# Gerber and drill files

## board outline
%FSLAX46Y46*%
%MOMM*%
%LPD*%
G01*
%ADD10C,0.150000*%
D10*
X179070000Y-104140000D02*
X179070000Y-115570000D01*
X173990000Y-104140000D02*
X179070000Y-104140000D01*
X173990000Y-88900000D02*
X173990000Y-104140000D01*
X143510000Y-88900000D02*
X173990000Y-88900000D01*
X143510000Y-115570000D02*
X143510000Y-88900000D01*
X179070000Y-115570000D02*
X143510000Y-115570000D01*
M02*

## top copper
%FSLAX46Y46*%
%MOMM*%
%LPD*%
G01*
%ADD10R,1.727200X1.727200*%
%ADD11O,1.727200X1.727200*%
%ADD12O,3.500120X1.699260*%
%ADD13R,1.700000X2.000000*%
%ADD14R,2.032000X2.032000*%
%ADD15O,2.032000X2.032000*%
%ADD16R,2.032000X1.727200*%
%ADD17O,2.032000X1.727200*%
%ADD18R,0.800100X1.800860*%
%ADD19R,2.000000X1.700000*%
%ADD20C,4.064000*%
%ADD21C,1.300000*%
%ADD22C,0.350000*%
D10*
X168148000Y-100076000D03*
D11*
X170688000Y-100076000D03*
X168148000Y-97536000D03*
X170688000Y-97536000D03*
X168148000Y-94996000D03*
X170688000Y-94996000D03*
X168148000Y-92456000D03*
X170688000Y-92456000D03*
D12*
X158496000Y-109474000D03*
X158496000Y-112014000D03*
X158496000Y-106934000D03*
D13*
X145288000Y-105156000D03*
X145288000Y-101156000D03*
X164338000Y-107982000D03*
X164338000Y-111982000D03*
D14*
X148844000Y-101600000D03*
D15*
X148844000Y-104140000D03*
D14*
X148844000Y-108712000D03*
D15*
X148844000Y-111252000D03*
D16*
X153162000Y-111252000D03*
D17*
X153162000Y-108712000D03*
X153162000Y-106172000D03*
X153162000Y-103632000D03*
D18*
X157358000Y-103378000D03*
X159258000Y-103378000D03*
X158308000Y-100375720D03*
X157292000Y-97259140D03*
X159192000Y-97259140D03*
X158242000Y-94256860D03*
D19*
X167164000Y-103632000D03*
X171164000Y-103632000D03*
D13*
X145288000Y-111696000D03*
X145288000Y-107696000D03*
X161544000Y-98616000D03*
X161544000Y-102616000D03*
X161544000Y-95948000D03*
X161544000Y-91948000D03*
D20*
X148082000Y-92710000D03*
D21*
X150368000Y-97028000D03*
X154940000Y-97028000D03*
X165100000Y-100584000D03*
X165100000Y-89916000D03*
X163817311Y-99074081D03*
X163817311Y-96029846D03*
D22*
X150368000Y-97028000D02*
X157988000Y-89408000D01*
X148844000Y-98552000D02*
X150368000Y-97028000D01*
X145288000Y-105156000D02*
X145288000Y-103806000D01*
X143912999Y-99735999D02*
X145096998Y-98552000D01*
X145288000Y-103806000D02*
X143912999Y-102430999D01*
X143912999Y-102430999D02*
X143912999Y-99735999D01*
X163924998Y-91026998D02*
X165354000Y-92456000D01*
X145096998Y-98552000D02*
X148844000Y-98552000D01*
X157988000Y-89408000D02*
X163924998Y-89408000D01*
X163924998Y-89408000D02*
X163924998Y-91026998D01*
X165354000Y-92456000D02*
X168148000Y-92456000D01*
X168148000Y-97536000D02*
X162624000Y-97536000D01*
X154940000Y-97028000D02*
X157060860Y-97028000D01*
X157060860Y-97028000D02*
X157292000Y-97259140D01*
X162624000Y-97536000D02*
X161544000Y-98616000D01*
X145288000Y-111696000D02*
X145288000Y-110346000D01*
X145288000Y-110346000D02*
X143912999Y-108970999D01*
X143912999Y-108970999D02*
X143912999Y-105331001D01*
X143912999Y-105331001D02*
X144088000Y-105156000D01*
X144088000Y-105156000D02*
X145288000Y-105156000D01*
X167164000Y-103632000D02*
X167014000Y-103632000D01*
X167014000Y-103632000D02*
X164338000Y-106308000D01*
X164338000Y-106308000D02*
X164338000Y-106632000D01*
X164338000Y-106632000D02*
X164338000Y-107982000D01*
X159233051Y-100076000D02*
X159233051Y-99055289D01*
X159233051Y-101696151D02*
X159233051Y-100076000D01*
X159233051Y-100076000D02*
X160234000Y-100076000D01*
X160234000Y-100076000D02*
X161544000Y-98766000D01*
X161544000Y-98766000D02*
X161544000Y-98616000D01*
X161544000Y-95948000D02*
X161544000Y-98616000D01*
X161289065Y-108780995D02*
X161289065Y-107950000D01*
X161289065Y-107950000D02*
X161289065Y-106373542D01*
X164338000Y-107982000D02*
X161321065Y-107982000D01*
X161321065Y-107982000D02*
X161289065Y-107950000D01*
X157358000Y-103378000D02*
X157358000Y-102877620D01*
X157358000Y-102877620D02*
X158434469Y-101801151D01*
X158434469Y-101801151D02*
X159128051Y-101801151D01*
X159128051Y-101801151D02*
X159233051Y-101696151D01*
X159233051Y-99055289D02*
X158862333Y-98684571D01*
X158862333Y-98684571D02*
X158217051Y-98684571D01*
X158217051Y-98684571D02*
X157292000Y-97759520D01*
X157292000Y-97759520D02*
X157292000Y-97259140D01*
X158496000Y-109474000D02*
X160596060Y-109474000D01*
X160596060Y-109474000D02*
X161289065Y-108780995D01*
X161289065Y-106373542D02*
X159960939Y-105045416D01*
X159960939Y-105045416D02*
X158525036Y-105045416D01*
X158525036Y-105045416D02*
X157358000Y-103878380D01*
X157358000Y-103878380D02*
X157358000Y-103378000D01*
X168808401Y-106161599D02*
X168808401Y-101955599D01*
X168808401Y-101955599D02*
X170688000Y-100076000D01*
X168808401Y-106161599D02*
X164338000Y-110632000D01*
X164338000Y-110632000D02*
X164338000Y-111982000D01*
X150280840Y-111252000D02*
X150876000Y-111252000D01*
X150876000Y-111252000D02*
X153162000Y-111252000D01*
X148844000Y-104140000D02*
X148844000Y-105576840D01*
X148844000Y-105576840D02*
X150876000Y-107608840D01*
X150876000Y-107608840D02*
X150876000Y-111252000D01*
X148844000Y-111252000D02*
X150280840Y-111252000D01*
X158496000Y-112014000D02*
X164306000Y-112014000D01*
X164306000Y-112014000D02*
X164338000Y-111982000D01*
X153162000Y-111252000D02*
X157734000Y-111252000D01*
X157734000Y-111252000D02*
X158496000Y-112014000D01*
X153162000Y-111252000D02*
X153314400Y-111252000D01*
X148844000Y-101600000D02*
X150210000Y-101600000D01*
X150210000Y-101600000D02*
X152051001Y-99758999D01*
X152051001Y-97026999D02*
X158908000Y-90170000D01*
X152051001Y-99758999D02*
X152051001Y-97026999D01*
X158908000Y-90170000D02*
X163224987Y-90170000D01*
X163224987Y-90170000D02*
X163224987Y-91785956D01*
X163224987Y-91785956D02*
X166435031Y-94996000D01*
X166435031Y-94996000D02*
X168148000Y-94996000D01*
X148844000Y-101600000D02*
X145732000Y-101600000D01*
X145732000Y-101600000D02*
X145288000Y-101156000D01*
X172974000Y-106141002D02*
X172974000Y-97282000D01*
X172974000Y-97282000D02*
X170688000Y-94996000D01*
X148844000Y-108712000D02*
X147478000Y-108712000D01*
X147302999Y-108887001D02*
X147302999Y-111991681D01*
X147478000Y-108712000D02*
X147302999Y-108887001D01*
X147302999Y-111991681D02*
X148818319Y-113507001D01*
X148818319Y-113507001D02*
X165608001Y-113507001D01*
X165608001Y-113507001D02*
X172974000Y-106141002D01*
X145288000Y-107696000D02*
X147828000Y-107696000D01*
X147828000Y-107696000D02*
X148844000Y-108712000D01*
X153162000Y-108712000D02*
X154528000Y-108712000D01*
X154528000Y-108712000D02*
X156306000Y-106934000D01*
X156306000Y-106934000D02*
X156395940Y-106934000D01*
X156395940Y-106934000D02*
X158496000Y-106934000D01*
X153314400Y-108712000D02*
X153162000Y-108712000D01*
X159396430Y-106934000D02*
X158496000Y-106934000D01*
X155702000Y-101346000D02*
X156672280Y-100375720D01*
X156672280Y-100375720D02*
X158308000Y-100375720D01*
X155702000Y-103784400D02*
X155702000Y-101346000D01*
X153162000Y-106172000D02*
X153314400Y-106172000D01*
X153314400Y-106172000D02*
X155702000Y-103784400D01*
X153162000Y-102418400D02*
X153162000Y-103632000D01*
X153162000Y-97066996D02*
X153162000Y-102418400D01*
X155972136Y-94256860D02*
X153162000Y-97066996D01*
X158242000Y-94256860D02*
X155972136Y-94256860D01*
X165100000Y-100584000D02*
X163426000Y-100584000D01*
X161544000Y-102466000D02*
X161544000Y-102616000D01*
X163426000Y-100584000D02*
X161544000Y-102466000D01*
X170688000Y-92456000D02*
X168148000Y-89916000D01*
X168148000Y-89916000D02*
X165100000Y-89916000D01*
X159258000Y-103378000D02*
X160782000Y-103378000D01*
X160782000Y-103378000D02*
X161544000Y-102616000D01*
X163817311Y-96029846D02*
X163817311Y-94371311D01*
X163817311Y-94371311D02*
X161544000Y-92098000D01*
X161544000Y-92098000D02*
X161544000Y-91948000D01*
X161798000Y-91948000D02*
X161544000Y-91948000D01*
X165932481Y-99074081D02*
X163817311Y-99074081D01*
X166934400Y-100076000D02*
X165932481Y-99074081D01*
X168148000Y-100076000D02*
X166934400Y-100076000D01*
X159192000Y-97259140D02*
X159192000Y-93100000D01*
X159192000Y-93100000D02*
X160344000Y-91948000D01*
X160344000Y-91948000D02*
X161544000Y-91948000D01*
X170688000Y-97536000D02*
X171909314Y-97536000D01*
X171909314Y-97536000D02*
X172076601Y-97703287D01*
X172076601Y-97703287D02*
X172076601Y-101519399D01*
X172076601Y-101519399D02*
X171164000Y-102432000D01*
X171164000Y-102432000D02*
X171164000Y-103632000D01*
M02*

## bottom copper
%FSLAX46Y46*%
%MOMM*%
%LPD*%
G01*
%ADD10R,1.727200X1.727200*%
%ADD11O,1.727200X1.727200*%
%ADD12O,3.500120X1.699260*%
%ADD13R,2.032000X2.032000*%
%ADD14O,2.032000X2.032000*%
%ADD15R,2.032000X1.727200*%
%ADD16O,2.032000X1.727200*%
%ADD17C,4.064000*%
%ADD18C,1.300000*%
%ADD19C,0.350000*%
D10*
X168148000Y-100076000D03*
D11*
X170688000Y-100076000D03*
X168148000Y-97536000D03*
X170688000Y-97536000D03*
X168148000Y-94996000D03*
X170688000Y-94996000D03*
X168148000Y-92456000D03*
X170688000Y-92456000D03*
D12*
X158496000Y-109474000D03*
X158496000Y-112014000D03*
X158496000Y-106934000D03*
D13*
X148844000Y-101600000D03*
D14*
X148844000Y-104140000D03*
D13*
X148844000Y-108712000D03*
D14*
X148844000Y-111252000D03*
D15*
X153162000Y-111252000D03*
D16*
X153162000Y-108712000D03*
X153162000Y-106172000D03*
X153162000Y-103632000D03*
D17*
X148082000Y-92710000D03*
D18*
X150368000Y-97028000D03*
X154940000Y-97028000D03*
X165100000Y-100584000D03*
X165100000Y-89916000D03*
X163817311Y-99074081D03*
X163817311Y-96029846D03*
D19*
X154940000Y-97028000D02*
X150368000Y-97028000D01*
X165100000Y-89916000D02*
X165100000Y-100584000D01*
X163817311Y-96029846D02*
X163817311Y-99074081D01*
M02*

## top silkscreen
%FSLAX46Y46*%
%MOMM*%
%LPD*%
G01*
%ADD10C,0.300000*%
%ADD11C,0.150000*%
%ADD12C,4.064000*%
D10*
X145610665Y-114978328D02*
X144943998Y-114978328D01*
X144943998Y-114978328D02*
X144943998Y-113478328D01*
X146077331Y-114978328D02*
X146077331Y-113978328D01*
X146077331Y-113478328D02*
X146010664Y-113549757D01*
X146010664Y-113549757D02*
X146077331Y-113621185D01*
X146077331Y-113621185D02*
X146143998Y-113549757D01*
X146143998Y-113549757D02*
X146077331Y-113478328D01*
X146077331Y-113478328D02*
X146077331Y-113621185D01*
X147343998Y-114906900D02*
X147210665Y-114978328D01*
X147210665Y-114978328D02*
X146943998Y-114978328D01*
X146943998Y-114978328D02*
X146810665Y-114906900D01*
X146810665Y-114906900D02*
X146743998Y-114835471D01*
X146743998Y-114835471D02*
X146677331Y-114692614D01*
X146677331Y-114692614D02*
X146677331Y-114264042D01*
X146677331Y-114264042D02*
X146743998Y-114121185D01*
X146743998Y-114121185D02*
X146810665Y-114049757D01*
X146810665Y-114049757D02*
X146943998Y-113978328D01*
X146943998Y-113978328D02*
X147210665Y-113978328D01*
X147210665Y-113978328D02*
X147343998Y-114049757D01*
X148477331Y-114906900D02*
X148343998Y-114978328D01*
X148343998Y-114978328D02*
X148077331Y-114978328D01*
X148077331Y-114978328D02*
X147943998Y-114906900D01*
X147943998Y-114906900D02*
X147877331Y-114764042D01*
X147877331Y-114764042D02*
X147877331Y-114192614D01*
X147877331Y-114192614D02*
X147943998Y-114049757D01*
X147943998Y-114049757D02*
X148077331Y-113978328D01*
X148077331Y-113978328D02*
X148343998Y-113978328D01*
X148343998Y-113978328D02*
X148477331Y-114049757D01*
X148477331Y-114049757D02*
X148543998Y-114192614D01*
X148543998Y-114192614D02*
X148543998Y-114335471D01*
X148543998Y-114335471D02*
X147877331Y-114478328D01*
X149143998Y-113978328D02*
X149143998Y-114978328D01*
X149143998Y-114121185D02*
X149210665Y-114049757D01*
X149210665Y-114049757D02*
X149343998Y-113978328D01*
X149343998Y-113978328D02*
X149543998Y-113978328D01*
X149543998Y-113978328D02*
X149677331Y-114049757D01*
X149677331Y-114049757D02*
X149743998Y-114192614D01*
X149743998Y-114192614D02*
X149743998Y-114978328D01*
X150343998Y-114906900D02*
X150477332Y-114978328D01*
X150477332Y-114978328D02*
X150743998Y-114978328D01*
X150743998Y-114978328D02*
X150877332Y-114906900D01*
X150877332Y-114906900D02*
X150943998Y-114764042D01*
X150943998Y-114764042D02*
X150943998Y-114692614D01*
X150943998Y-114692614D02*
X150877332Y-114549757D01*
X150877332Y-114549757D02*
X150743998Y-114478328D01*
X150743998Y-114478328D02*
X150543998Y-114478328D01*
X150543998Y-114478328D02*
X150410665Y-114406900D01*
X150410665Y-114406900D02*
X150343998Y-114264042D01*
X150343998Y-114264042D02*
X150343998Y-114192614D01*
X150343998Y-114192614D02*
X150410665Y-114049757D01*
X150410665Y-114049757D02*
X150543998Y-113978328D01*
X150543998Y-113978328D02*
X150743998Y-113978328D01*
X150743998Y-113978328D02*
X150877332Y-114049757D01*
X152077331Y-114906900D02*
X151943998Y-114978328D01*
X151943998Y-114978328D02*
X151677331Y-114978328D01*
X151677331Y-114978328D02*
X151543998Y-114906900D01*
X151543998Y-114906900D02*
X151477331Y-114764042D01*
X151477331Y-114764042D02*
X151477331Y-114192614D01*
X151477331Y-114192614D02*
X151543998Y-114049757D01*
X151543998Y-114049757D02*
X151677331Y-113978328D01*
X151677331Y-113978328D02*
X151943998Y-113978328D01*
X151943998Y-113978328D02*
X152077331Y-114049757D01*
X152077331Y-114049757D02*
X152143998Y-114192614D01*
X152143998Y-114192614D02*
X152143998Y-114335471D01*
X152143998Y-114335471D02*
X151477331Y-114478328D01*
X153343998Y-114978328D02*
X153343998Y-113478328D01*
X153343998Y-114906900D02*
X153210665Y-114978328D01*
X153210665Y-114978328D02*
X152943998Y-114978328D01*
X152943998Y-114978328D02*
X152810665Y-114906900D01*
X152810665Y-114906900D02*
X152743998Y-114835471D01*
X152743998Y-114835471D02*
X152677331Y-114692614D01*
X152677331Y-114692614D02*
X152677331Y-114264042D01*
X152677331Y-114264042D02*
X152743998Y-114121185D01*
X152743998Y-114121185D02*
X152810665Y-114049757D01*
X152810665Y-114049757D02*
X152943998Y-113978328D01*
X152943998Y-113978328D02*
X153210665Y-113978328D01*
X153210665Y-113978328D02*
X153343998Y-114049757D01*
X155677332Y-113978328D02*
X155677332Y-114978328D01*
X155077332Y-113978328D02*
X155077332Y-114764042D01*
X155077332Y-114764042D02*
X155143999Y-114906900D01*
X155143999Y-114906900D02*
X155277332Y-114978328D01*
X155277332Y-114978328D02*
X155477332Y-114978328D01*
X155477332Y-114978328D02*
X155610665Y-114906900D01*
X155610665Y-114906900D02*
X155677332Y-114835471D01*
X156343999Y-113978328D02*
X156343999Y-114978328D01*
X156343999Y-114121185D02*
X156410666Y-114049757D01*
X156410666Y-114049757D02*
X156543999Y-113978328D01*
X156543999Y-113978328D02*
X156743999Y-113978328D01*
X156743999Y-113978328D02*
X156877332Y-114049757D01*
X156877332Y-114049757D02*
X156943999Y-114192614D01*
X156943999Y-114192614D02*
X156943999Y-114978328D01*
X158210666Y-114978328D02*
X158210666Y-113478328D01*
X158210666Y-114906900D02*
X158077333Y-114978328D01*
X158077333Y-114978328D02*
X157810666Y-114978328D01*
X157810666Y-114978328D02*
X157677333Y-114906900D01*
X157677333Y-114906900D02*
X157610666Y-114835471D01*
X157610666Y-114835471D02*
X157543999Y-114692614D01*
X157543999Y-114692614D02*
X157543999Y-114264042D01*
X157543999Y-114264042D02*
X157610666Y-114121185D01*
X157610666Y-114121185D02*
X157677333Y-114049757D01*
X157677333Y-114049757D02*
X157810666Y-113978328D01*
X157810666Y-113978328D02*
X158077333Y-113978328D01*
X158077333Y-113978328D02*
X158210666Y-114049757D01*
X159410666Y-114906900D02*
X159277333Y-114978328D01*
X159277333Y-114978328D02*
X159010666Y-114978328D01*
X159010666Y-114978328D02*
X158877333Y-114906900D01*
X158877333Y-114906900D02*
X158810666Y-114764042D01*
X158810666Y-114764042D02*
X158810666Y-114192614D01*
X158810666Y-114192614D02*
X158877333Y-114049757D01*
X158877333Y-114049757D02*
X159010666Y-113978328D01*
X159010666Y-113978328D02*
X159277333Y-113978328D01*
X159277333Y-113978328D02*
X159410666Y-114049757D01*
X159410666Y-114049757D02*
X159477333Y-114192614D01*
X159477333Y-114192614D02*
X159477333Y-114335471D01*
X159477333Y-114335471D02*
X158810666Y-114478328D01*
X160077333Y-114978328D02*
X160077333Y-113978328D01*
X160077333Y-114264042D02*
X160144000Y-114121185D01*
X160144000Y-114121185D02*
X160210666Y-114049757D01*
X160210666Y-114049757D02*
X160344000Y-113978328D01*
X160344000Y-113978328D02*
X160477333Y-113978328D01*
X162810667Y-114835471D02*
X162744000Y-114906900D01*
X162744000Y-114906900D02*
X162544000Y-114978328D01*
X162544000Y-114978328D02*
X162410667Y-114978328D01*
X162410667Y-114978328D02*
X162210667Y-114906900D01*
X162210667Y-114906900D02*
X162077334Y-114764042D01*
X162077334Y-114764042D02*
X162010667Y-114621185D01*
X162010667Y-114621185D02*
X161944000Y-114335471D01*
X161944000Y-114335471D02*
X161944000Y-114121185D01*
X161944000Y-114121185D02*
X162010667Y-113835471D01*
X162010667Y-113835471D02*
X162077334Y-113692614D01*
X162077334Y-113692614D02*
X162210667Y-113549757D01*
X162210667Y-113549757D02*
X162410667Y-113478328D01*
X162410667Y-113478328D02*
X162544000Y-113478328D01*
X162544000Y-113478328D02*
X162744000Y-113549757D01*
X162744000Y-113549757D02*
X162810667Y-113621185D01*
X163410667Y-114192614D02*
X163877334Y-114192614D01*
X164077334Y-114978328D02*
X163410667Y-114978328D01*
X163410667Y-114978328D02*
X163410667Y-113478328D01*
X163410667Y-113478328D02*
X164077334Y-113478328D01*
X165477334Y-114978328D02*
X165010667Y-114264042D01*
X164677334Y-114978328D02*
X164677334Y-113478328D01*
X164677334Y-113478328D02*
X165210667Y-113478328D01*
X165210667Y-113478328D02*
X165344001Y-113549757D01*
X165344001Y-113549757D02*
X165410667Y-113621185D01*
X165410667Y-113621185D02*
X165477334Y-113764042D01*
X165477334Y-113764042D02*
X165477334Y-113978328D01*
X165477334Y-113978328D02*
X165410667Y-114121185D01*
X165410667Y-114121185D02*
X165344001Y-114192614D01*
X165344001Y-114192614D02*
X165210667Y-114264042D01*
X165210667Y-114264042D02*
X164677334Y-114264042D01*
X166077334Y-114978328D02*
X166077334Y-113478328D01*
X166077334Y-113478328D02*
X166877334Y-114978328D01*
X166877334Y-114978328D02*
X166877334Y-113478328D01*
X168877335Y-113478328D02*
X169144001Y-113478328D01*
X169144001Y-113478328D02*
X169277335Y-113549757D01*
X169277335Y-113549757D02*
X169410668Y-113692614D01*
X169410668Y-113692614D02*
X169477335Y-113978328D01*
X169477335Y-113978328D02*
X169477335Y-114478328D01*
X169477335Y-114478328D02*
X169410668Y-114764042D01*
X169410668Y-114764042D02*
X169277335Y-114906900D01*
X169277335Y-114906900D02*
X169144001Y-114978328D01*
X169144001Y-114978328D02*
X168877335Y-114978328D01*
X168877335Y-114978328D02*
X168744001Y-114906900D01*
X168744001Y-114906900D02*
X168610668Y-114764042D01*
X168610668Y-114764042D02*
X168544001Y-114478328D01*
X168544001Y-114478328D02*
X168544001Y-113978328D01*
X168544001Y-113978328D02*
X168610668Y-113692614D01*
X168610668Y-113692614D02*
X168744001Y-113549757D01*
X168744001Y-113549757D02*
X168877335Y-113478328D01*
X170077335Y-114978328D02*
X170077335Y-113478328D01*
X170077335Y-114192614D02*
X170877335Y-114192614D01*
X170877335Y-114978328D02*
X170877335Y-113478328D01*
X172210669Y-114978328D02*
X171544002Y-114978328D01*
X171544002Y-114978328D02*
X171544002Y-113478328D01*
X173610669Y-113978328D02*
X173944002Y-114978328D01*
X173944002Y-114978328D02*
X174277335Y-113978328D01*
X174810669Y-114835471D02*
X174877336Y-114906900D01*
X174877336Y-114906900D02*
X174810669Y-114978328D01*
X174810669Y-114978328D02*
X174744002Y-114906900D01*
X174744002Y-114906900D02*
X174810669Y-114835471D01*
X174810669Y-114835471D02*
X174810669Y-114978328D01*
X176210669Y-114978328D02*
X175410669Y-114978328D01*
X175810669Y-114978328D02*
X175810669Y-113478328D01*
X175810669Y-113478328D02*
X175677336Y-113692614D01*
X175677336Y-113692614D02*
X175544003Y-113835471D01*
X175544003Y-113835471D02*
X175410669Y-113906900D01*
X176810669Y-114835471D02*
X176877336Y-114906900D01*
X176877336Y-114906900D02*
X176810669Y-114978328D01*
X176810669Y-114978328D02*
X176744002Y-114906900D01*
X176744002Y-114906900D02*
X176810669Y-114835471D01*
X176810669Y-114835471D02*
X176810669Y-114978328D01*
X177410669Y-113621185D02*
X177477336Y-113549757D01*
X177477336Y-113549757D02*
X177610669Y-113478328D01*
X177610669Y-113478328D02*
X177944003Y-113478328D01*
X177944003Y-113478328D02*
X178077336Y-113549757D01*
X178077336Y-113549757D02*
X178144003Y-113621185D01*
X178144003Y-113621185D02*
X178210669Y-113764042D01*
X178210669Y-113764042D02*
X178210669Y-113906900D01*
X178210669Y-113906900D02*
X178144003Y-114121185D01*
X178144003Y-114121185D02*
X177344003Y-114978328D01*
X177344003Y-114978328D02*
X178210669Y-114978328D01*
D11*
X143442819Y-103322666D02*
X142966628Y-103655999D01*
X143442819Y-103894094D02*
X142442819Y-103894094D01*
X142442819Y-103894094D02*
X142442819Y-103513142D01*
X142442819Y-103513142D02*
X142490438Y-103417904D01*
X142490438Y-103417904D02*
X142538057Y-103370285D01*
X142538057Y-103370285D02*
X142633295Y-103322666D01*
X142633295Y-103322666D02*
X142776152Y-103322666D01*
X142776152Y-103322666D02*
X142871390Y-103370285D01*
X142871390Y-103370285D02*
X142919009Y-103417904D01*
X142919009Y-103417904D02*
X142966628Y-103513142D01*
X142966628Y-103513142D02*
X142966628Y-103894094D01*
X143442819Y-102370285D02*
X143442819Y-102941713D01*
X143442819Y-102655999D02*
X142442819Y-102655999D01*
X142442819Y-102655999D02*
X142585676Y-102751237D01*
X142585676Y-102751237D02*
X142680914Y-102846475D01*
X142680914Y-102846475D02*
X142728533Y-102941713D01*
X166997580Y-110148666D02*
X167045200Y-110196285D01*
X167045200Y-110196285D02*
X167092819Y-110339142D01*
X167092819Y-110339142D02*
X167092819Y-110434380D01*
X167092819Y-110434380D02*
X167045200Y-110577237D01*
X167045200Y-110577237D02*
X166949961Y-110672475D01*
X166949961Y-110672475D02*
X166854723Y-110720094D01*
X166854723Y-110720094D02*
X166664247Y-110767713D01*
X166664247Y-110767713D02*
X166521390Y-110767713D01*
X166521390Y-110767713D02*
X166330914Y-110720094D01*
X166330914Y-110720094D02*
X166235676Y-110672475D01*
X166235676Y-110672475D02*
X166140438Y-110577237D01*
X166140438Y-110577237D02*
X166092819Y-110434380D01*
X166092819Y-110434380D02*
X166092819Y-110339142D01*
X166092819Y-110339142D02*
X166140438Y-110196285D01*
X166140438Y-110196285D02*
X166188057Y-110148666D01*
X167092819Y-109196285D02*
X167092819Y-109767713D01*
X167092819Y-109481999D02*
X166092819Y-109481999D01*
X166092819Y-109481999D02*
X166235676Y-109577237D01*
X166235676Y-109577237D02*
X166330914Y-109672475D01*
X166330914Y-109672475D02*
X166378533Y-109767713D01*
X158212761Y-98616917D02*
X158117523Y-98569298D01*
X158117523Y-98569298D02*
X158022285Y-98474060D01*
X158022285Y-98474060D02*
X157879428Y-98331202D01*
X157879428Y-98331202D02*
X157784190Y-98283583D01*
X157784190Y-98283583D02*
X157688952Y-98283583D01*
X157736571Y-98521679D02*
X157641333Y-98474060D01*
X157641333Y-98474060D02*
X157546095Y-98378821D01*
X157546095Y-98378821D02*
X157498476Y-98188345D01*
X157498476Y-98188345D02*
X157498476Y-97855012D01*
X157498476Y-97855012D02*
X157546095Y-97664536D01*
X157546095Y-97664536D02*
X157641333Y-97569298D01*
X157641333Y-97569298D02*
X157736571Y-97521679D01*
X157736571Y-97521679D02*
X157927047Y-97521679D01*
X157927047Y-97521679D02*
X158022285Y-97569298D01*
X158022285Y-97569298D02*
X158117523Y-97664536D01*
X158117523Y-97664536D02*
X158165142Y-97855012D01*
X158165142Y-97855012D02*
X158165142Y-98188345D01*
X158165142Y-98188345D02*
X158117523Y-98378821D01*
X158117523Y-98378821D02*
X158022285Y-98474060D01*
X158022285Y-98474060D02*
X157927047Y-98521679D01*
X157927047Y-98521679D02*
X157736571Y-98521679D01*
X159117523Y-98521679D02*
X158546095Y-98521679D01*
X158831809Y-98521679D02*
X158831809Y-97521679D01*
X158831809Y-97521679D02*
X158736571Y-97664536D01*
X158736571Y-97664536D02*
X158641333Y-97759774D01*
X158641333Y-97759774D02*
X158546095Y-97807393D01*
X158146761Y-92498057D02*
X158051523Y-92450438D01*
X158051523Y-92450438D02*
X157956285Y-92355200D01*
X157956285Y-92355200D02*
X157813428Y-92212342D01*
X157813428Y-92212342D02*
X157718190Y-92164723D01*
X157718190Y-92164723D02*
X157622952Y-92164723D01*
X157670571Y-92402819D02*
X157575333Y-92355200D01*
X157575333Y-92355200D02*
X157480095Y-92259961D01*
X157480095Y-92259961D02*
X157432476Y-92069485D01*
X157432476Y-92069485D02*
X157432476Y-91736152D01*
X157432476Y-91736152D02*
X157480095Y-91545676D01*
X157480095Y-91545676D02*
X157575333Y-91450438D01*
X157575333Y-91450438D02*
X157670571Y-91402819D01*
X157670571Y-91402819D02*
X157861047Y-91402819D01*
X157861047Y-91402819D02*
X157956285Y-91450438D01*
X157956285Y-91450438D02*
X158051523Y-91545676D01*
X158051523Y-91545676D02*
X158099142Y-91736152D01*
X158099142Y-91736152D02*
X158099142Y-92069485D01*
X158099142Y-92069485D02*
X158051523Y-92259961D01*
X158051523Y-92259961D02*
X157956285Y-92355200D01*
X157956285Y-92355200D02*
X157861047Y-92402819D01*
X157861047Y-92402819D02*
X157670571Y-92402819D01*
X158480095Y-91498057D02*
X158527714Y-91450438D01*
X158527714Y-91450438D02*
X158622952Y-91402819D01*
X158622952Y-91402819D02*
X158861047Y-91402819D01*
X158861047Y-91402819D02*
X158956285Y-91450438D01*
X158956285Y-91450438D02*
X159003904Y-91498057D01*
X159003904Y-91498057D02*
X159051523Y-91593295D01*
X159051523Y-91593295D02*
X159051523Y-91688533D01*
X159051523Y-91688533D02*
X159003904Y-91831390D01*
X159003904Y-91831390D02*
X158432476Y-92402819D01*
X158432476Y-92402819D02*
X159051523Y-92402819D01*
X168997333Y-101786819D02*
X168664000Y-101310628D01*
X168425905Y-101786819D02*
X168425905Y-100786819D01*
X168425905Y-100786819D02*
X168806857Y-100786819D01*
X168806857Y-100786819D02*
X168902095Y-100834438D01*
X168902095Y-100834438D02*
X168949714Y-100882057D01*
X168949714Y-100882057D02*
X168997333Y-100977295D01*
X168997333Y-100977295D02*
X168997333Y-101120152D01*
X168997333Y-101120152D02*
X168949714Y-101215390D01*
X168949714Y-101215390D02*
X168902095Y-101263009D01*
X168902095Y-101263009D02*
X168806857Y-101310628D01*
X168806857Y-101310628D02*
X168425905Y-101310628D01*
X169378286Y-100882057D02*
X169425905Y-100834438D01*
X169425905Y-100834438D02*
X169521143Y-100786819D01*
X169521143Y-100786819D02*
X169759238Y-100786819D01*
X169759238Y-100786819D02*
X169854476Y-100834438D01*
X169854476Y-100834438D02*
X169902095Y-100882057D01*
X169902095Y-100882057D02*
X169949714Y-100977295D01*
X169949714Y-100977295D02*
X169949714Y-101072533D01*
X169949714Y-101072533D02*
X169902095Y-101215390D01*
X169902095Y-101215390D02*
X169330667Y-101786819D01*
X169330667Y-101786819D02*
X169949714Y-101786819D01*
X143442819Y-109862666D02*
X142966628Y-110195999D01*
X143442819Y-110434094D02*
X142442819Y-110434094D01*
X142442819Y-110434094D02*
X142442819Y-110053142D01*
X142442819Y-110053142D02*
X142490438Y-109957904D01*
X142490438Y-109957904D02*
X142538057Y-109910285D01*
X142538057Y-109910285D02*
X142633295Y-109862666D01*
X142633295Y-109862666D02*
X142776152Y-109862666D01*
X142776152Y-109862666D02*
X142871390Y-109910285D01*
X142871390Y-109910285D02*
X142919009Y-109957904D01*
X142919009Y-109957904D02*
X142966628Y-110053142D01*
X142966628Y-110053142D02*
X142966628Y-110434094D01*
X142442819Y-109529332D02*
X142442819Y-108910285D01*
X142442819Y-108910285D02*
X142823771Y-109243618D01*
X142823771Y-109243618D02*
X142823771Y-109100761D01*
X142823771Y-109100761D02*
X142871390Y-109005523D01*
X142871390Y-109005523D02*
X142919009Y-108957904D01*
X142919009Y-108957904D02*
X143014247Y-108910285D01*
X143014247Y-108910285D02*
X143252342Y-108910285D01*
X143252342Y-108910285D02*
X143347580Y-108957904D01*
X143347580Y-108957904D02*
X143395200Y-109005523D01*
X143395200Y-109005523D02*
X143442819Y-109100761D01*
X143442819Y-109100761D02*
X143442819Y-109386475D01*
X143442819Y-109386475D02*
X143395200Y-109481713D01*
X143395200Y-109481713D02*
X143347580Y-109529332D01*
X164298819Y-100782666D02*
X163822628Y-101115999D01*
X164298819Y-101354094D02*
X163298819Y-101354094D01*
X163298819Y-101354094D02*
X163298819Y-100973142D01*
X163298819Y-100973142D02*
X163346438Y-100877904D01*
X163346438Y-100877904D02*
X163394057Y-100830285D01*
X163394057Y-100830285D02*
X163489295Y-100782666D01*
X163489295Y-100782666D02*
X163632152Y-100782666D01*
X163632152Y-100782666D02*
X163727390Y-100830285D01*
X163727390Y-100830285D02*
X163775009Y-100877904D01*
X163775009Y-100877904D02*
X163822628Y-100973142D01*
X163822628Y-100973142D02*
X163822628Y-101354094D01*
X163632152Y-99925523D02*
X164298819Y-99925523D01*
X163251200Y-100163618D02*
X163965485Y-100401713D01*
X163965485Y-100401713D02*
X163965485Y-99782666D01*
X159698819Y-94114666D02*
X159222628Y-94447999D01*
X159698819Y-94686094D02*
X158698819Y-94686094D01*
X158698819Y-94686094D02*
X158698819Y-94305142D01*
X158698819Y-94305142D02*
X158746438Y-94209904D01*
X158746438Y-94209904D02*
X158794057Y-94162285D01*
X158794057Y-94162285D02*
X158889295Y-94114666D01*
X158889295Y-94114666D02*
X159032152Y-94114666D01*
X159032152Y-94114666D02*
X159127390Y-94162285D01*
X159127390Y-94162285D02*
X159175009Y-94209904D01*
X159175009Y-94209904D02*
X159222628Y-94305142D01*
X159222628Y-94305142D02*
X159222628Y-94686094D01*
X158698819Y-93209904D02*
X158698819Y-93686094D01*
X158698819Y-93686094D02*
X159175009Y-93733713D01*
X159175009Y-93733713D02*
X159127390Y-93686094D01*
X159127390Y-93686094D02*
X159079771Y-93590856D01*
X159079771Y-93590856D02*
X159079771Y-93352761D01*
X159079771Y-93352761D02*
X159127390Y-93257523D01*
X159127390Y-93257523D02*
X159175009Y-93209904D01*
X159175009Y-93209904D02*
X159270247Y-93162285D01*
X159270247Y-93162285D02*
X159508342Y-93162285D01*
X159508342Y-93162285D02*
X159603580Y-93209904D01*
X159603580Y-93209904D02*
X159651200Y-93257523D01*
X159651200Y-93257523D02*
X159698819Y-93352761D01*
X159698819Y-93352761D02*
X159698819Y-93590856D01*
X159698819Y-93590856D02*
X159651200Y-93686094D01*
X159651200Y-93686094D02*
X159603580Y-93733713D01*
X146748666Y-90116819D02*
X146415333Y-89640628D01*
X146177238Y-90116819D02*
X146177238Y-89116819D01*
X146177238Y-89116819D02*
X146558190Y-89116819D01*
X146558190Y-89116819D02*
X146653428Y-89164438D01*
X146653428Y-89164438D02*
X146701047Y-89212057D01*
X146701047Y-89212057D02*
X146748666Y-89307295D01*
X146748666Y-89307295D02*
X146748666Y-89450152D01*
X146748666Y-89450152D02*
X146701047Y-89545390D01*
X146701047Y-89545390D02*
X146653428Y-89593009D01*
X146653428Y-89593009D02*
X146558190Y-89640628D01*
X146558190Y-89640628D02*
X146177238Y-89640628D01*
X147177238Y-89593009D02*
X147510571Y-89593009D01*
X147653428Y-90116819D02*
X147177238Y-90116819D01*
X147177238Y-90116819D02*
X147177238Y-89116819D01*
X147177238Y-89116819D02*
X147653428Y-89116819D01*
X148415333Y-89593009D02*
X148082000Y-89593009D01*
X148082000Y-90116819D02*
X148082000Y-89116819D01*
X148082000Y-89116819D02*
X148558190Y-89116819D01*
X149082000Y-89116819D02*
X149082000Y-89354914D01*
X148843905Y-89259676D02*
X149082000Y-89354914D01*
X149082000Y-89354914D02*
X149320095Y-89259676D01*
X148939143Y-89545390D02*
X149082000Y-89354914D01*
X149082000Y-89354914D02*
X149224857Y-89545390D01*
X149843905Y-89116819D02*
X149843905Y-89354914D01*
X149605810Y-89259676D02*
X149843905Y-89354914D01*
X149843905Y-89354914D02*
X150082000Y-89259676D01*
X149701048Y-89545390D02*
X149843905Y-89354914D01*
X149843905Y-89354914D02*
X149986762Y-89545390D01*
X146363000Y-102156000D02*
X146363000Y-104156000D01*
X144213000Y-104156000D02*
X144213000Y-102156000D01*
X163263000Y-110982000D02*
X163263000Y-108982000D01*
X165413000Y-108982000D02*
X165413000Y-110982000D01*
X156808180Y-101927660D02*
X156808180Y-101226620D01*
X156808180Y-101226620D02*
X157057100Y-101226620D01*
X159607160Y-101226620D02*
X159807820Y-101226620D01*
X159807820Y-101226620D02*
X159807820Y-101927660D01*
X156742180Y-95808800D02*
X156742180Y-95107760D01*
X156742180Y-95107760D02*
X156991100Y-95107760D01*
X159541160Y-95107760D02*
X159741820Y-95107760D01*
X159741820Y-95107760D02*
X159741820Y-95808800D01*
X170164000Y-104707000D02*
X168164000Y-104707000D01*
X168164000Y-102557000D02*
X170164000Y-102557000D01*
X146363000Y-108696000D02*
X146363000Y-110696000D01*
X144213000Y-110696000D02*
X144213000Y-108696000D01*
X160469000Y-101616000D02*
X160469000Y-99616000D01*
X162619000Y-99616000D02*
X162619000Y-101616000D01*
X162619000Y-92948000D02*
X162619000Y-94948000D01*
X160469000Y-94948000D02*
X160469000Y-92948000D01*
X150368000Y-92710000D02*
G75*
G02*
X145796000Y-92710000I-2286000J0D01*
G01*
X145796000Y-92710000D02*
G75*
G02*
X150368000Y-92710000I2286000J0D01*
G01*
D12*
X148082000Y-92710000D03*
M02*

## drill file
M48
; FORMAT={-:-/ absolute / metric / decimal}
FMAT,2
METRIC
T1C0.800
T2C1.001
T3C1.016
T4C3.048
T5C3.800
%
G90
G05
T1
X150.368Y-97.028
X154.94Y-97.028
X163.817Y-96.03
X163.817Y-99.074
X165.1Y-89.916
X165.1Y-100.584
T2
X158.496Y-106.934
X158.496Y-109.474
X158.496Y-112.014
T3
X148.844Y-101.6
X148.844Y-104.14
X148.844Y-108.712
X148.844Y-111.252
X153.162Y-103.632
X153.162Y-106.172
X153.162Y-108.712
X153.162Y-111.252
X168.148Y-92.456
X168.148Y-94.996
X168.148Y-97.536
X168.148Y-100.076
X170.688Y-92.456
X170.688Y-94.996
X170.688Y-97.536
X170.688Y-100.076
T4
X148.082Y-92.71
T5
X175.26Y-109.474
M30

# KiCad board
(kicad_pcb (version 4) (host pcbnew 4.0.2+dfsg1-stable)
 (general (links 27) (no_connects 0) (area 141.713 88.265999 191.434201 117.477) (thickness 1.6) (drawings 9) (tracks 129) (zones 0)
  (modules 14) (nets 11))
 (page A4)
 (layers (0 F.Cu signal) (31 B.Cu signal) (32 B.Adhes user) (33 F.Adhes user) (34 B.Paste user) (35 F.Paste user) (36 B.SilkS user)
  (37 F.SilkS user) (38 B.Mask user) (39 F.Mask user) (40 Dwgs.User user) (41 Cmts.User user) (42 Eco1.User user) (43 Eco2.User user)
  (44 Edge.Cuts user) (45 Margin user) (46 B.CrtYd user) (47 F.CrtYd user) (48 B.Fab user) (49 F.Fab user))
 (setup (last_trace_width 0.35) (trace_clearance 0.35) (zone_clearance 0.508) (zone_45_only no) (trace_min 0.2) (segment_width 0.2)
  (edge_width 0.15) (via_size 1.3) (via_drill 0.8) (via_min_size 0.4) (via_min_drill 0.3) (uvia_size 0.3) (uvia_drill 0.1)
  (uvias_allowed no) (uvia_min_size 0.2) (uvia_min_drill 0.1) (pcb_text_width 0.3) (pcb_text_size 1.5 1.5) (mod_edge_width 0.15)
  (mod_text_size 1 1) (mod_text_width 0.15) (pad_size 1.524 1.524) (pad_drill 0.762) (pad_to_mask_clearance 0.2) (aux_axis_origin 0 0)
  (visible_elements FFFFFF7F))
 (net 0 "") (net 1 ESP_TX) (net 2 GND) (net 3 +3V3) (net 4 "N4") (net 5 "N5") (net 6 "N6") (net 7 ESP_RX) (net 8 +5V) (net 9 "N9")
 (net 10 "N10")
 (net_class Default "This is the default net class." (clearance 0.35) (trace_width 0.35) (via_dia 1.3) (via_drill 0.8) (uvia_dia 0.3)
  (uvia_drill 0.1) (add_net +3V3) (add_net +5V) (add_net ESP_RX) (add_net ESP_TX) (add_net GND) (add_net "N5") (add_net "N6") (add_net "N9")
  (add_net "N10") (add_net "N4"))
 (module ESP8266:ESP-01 (layer B.Cu) (at 168.148 100.076)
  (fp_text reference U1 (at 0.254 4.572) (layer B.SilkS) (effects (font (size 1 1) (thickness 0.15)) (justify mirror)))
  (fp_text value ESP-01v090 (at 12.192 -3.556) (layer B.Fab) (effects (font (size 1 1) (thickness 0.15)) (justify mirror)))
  (pad 1 thru_hole rect (at 0 0) (size 1.7272 1.7272) (drill 1.016) (layers *.Cu *.Mask B.SilkS) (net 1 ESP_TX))
  (pad 2 thru_hole oval (at 2.54 0) (size 1.7272 1.7272) (drill 1.016) (layers *.Cu *.Mask B.SilkS) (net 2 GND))
  (pad 3 thru_hole oval (at 0 -2.54) (size 1.7272 1.7272) (drill 1.016) (layers *.Cu *.Mask B.SilkS) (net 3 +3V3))
  (pad 4 thru_hole oval (at 2.54 -2.54) (size 1.7272 1.7272) (drill 1.016) (layers *.Cu *.Mask B.SilkS) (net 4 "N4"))
  (pad 5 thru_hole oval (at 0 -5.08) (size 1.7272 1.7272) (drill 1.016) (layers *.Cu *.Mask B.SilkS) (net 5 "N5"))
  (pad 6 thru_hole oval (at 2.54 -5.08) (size 1.7272 1.7272) (drill 1.016) (layers *.Cu *.Mask B.SilkS) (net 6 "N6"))
  (pad 7 thru_hole oval (at 0 -7.62) (size 1.7272 1.7272) (drill 1.016) (layers *.Cu *.Mask B.SilkS) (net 3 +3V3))
  (pad 8 thru_hole oval (at 2.54 -7.62) (size 1.7272 1.7272) (drill 1.016) (layers *.Cu *.Mask B.SilkS) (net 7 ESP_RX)))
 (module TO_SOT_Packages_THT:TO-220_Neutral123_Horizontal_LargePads (layer B.Cu) (at 158.496 109.474 90)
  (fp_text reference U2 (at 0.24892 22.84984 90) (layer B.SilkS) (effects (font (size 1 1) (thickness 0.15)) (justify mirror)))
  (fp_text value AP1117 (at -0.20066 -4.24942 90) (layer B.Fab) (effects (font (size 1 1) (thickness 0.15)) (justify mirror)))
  (pad 2 thru_hole oval (at 0 0) (size 3.50012 1.69926) (drill 1.00076) (layers *.Cu *.Mask B.SilkS) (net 3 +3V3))
  (pad 1 thru_hole oval (at -2.54 0) (size 3.50012 1.69926) (drill 1.00076) (layers *.Cu *.Mask B.SilkS) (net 2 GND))
  (pad 3 thru_hole oval (at 2.54 0) (size 3.50012 1.69926) (drill 1.00076) (layers *.Cu *.Mask B.SilkS) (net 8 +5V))
  (pad "" np_thru_hole circle (at 0 16.764) (size 3.79984 3.79984) (drill 3.79984) (layers *.Cu *.Mask B.SilkS)))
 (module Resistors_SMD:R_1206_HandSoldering (layer F.Cu) (at 145.288 103.156 90)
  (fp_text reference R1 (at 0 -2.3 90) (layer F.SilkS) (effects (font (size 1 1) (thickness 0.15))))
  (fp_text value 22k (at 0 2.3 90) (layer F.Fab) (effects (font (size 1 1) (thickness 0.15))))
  (fp_line (start 1 1.075) (end -1 1.075) (layer F.SilkS) (width 0.15))
  (fp_line (start -1 -1.075) (end 1 -1.075) (layer F.SilkS) (width 0.15))
  (pad 1 smd rect (at -2 0 90) (size 2 1.7) (layers F.Cu F.Paste F.Mask) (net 3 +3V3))
  (pad 2 smd rect (at 2 0 90) (size 2 1.7) (layers F.Cu F.Paste F.Mask) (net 5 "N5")))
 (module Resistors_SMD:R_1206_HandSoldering (layer F.Cu) (at 164.338 109.982 270)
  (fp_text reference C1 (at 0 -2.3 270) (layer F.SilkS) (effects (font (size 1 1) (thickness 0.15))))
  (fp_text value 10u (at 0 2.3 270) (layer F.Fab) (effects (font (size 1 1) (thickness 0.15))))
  (fp_line (start 1 1.075) (end -1 1.075) (layer F.SilkS) (width 0.15))
  (fp_line (start -1 -1.075) (end 1 -1.075) (layer F.SilkS) (width 0.15))
  (pad 1 smd rect (at -2 0 270) (size 2 1.7) (layers F.Cu F.Paste F.Mask) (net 3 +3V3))
  (pad 2 smd rect (at 2 0 270) (size 2 1.7) (layers F.Cu F.Paste F.Mask) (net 2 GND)))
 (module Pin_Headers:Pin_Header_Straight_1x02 (layer B.Cu) (at 148.844 101.6 180)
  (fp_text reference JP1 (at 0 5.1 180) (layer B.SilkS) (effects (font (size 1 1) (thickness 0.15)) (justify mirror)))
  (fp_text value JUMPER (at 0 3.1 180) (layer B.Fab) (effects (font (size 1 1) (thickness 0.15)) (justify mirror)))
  (pad 1 thru_hole rect (at 0 0 180) (size 2.032 2.032) (drill 1.016) (layers *.Cu *.Mask B.SilkS) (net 5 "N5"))
  (pad 2 thru_hole oval (at 0 -2.54 180) (size 2.032 2.032) (drill 1.016) (layers *.Cu *.Mask B.SilkS) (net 2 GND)))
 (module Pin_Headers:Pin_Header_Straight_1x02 (layer B.Cu) (at 148.844 108.712 180)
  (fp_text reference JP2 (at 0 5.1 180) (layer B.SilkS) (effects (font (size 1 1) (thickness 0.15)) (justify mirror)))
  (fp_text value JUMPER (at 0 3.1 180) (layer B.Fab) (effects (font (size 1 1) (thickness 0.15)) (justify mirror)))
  (pad 1 thru_hole rect (at 0 0 180) (size 2.032 2.032) (drill 1.016) (layers *.Cu *.Mask B.SilkS) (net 6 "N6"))
  (pad 2 thru_hole oval (at 0 -2.54 180) (size 2.032 2.032) (drill 1.016) (layers *.Cu *.Mask B.SilkS) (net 2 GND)))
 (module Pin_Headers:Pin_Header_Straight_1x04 (layer B.Cu) (at 153.162 111.252)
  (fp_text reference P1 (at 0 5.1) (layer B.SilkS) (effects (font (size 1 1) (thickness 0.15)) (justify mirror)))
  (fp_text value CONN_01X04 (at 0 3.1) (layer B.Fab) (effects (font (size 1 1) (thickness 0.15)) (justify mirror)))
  (pad 1 thru_hole rect (at 0 0) (size 2.032 1.7272) (drill 1.016) (layers *.Cu *.Mask B.SilkS) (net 2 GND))
  (pad 2 thru_hole oval (at 0 -2.54) (size 2.032 1.7272) (drill 1.016) (layers *.Cu *.Mask B.SilkS) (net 8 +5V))
  (pad 3 thru_hole oval (at 0 -5.08) (size 2.032 1.7272) (drill 1.016) (layers *.Cu *.Mask B.SilkS) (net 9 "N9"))
  (pad 4 thru_hole oval (at 0 -7.62) (size 2.032 1.7272) (drill 1.016) (layers *.Cu *.Mask B.SilkS) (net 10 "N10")))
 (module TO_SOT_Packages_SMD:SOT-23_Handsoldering (layer F.Cu) (at 158.308 101.87686)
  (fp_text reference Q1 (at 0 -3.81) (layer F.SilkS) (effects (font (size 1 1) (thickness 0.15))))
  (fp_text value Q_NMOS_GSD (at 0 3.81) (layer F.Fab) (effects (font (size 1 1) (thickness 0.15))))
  (fp_line (start -1.49982 0.0508) (end -1.49982 -0.65024) (layer F.SilkS) (width 0.15))
  (fp_line (start -1.49982 -0.65024) (end -1.2509 -0.65024) (layer F.SilkS) (width 0.15))
  (fp_line (start 1.29916 -0.65024) (end 1.49982 -0.65024) (layer F.SilkS) (width 0.15))
  (fp_line (start 1.49982 -0.65024) (end 1.49982 0.0508) (layer F.SilkS) (width 0.15))
  (pad 1 smd rect (at -0.95 1.50114) (size 0.8001 1.80086) (layers F.Cu F.Paste F.Mask) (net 3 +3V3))
  (pad 2 smd rect (at 0.95 1.50114) (size 0.8001 1.80086) (layers F.Cu F.Paste F.Mask) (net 7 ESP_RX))
  (pad 3 smd rect (at 0 -1.50114) (size 0.8001 1.80086) (layers F.Cu F.Paste F.Mask) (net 9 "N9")))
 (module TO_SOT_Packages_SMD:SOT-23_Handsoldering (layer F.Cu) (at 158.242 95.758)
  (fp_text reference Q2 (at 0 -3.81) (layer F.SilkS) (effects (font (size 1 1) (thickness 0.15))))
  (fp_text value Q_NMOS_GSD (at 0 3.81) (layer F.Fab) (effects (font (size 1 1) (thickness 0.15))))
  (fp_line (start -1.49982 0.0508) (end -1.49982 -0.65024) (layer F.SilkS) (width 0.15))
  (fp_line (start -1.49982 -0.65024) (end -1.2509 -0.65024) (layer F.SilkS) (width 0.15))
  (fp_line (start 1.29916 -0.65024) (end 1.49982 -0.65024) (layer F.SilkS) (width 0.15))
  (fp_line (start 1.49982 -0.65024) (end 1.49982 0.0508) (layer F.SilkS) (width 0.15))
  (pad 1 smd rect (at -0.95 1.50114) (size 0.8001 1.80086) (layers F.Cu F.Paste F.Mask) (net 3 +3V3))
  (pad 2 smd rect (at 0.95 1.50114) (size 0.8001 1.80086) (layers F.Cu F.Paste F.Mask) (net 1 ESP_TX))
  (pad 3 smd rect (at 0 -1.50114) (size 0.8001 1.80086) (layers F.Cu F.Paste F.Mask) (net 10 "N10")))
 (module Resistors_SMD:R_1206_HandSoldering (layer F.Cu) (at 169.164 103.632)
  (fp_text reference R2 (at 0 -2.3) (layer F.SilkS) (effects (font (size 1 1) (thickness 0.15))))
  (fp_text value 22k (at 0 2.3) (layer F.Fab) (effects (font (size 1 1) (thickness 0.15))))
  (fp_line (start 1 1.075) (end -1 1.075) (layer F.SilkS) (width 0.15))
  (fp_line (start -1 -1.075) (end 1 -1.075) (layer F.SilkS) (width 0.15))
  (pad 1 smd rect (at -2 0) (size 2 1.7) (layers F.Cu F.Paste F.Mask) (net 3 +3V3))
  (pad 2 smd rect (at 2 0) (size 2 1.7) (layers F.Cu F.Paste F.Mask) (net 4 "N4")))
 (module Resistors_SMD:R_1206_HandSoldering (layer F.Cu) (at 145.288 109.696 90)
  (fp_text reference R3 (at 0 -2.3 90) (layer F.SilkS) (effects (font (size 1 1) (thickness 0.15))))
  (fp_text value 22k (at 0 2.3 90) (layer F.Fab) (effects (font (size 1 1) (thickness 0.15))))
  (fp_line (start 1 1.075) (end -1 1.075) (layer F.SilkS) (width 0.15))
  (fp_line (start -1 -1.075) (end 1 -1.075) (layer F.SilkS) (width 0.15))
  (pad 1 smd rect (at -2 0 90) (size 2 1.7) (layers F.Cu F.Paste F.Mask) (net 3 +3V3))
  (pad 2 smd rect (at 2 0 90) (size 2 1.7) (layers F.Cu F.Paste F.Mask) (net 6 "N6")))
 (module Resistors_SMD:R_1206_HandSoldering (layer F.Cu) (at 161.544 100.616 270)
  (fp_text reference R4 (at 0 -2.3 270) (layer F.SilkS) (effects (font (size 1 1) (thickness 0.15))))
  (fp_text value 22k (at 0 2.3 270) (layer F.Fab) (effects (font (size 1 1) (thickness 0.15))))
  (fp_line (start 1 1.075) (end -1 1.075) (layer F.SilkS) (width 0.15))
  (fp_line (start -1 -1.075) (end 1 -1.075) (layer F.SilkS) (width 0.15))
  (pad 1 smd rect (at -2 0 270) (size 2 1.7) (layers F.Cu F.Paste F.Mask) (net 3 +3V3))
  (pad 2 smd rect (at 2 0 270) (size 2 1.7) (layers F.Cu F.Paste F.Mask) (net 7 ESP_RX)))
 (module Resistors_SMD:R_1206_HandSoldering (layer F.Cu) (at 161.544 93.948 90)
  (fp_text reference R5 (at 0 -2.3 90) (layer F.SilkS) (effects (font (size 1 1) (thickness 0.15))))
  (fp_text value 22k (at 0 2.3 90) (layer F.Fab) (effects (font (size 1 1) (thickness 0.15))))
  (fp_line (start 1 1.075) (end -1 1.075) (layer F.SilkS) (width 0.15))
  (fp_line (start -1 -1.075) (end 1 -1.075) (layer F.SilkS) (width 0.15))
  (pad 1 smd rect (at -2 0 90) (size 2 1.7) (layers F.Cu F.Paste F.Mask) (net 3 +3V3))
  (pad 2 smd rect (at 2 0 90) (size 2 1.7) (layers F.Cu F.Paste F.Mask) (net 1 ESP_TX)))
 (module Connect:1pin (layer F.Cu) (at 148.082 92.71)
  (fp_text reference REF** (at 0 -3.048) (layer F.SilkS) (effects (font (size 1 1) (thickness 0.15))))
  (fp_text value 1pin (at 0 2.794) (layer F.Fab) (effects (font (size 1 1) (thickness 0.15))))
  (fp_circle (center 0 0) (end 0 -2.286) (layer F.SilkS) (width 0.15))
  (pad 1 thru_hole circle (at 0 0) (size 4.064 4.064) (drill 3.048) (layers *.Cu *.Mask F.SilkS)))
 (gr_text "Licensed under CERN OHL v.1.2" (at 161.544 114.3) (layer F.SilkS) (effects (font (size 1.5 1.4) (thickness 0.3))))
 (gr_line (start 179.07 104.14) (end 179.07 115.57) (layer Edge.Cuts) (width 0.15))
 (gr_line (start 173.99 104.14) (end 179.07 104.14) (layer Edge.Cuts) (width 0.15))
 (gr_line (start 173.99 88.9) (end 173.99 104.14) (layer Edge.Cuts) (width 0.15))
 (gr_line (start 143.51 88.9) (end 173.99 88.9) (layer Edge.Cuts) (width 0.15))
 (gr_line (start 143.51 115.57) (end 143.51 88.9) (layer Edge.Cuts) (width 0.15))
 (gr_line (start 179.07 115.57) (end 143.51 115.57) (layer Edge.Cuts) (width 0.15))
 (segment (start 150.368 97.028) (end 157.988 89.408) (width 0.35) (layer F.Cu) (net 3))
 (segment (start 148.844 98.552) (end 150.368 97.028) (width 0.35) (layer F.Cu) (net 3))
 (segment (start 145.288 105.156) (end 145.288 103.806) (width 0.35) (layer F.Cu) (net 3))
 (segment (start 143.912999 99.735999) (end 145.096998 98.552) (width 0.35) (layer F.Cu) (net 3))
 (segment (start 145.288 103.806) (end 143.912999 102.430999) (width 0.35) (layer F.Cu) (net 3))
 (segment (start 143.912999 102.430999) (end 143.912999 99.735999) (width 0.35) (layer F.Cu) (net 3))
 (segment (start 163.924998 91.026998) (end 165.354 92.456) (width 0.35) (layer F.Cu) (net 3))
 (segment (start 145.096998 98.552) (end 148.844 98.552) (width 0.35) (layer F.Cu) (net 3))
 (segment (start 157.988 89.408) (end 163.924998 89.408) (width 0.35) (layer F.Cu) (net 3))
 (segment (start 163.924998 89.408) (end 163.924998 91.026998) (width 0.35) (layer F.Cu) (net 3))
 (segment (start 165.354 92.456) (end 168.148 92.456) (width 0.35) (layer F.Cu) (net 3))
 (segment (start 168.148 97.536) (end 162.624 97.536) (width 0.35) (layer F.Cu) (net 3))
 (segment (start 154.94 97.028) (end 157.06086 97.028) (width 0.35) (layer F.Cu) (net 3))
 (segment (start 157.06086 97.028) (end 157.292 97.25914) (width 0.35) (layer F.Cu) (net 3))
 (segment (start 154.94 97.028) (end 150.368 97.028) (width 0.35) (layer B.Cu) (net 3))
 (via (at 150.368 97.028) (size 1.3) (drill 0.8) (layers F.Cu B.Cu) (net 3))
 (via (at 154.94 97.028) (size 1.3) (drill 0.8) (layers F.Cu B.Cu) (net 3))
 (segment (start 162.624 97.536) (end 161.544 98.616) (width 0.35) (layer F.Cu) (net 3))
 (segment (start 145.288 111.696) (end 145.288 110.346) (width 0.35) (layer F.Cu) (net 3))
 (segment (start 145.288 110.346) (end 143.912999 108.970999) (width 0.35) (layer F.Cu) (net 3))
 (segment (start 143.912999 108.970999) (end 143.912999 105.331001) (width 0.35) (layer F.Cu) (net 3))
 (segment (start 143.912999 105.331001) (end 144.088 105.156) (width 0.35) (layer F.Cu) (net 3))
 (segment (start 144.088 105.156) (end 145.288 105.156) (width 0.35) (layer F.Cu) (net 3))
 (segment (start 167.164 103.632) (end 167.014 103.632) (width 0.35) (layer F.Cu) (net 3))
 (segment (start 167.014 103.632) (end 164.338 106.308) (width 0.35) (layer F.Cu) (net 3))
 (segment (start 164.338 106.308) (end 164.338 106.632) (width 0.35) (layer F.Cu) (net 3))
 (segment (start 164.338 106.632) (end 164.338 107.982) (width 0.35) (layer F.Cu) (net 3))
 (segment (start 159.233051 100.076) (end 159.233051 99.055289) (width 0.35) (layer F.Cu) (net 3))
 (segment (start 159.233051 101.696151) (end 159.233051 100.076) (width 0.35) (layer F.Cu) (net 3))
 (segment (start 159.233051 100.076) (end 160.234 100.076) (width 0.35) (layer F.Cu) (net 3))
 (segment (start 160.234 100.076) (end 161.544 98.766) (width 0.35) (layer F.Cu) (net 3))
 (segment (start 161.544 98.766) (end 161.544 98.616) (width 0.35) (layer F.Cu) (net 3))
 (segment (start 161.544 95.948) (end 161.544 98.616) (width 0.35) (layer F.Cu) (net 3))
 (segment (start 161.289065 108.780995) (end 161.289065 107.95) (width 0.35) (layer F.Cu) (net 3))
 (segment (start 161.289065 107.95) (end 161.289065 106.373542) (width 0.35) (layer F.Cu) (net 3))
 (segment (start 164.338 107.982) (end 161.321065 107.982) (width 0.35) (layer F.Cu) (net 3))
 (segment (start 161.321065 107.982) (end 161.289065 107.95) (width 0.35) (layer F.Cu) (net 3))
 (segment (start 157.358 103.378) (end 157.358 102.87762) (width 0.35) (layer F.Cu) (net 3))
 (segment (start 157.358 102.87762) (end 158.434469 101.801151) (width 0.35) (layer F.Cu) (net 3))
 (segment (start 158.434469 101.801151) (end 159.128051 101.801151) (width 0.35) (layer F.Cu) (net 3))
 (segment (start 159.128051 101.801151) (end 159.233051 101.696151) (width 0.35) (layer F.Cu) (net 3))
 (segment (start 159.233051 99.055289) (end 158.862333 98.684571) (width 0.35) (layer F.Cu) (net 3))
 (segment (start 158.862333 98.684571) (end 158.217051 98.684571) (width 0.35) (layer F.Cu) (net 3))
 (segment (start 158.217051 98.684571) (end 157.292 97.75952) (width 0.35) (layer F.Cu) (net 3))
 (segment (start 157.292 97.75952) (end 157.292 97.25914) (width 0.35) (layer F.Cu) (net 3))
 (segment (start 158.496 109.474) (end 160.59606 109.474) (width 0.35) (layer F.Cu) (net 3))
 (segment (start 160.59606 109.474) (end 161.289065 108.780995) (width 0.35) (layer F.Cu) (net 3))
 (segment (start 161.289065 106.373542) (end 159.960939 105.045416) (width 0.35) (layer F.Cu) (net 3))
 (segment (start 159.960939 105.045416) (end 158.525036 105.045416) (width 0.35) (layer F.Cu) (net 3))
 (segment (start 158.525036 105.045416) (end 157.358 103.87838) (width 0.35) (layer F.Cu) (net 3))
 (segment (start 157.358 103.87838) (end 157.358 103.378) (width 0.35) (layer F.Cu) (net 3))
 (segment (start 168.808401 106.161599) (end 168.808401 101.955599) (width 0.35) (layer F.Cu) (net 2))
 (segment (start 168.808401 101.955599) (end 170.688 100.076) (width 0.35) (layer F.Cu) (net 2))
 (segment (start 168.808401 106.161599) (end 164.338 110.632) (width 0.35) (layer F.Cu) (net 2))
 (segment (start 164.338 110.632) (end 164.338 111.982) (width 0.35) (layer F.Cu) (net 2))
 (segment (start 150.28084 111.252) (end 150.876 111.252) (width 0.35) (layer F.Cu) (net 2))
 (segment (start 150.876 111.252) (end 153.162 111.252) (width 0.35) (layer F.Cu) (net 2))
 (segment (start 148.844 104.14) (end 148.844 105.57684) (width 0.35) (layer F.Cu) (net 2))
 (segment (start 148.844 105.57684) (end 150.876 107.60884) (width 0.35) (layer F.Cu) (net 2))
 (segment (start 150.876 107.60884) (end 150.876 111.252) (width 0.35) (layer F.Cu) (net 2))
 (segment (start 148.844 111.252) (end 150.28084 111.252) (width 0.35) (layer F.Cu) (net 2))
 (segment (start 158.496 112.014) (end 164.306 112.014) (width 0.35) (layer F.Cu) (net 2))
 (segment (start 164.306 112.014) (end 164.338 111.982) (width 0.35) (layer F.Cu) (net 2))
 (segment (start 153.162 111.252) (end 157.734 111.252) (width 0.35) (layer F.Cu) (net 2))
 (segment (start 157.734 111.252) (end 158.496 112.014) (width 0.35) (layer F.Cu) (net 2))
 (segment (start 153.162 111.252) (end 153.3144 111.252) (width 0.35) (layer F.Cu) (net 2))
 (segment (start 148.844 101.6) (end 150.21 101.6) (width 0.35) (layer F.Cu) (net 5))
 (segment (start 150.21 101.6) (end 152.051001 99.758999) (width 0.35) (layer F.Cu) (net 5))
 (segment (start 152.051001 97.026999) (end 158.908 90.17) (width 0.35) (layer F.Cu) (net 5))
 (segment (start 152.051001 99.758999) (end 152.051001 97.026999) (width 0.35) (layer F.Cu) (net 5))
 (segment (start 158.908 90.17) (end 163.224987 90.17) (width 0.35) (layer F.Cu) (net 5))
 (segment (start 163.224987 90.17) (end 163.224987 91.785956) (width 0.35) (layer F.Cu) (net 5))
 (segment (start 163.224987 91.785956) (end 166.435031 94.996) (width 0.35) (layer F.Cu) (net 5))
 (segment (start 166.435031 94.996) (end 168.148 94.996) (width 0.35) (layer F.Cu) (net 5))
 (segment (start 148.844 101.6) (end 145.732 101.6) (width 0.35) (layer F.Cu) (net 5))
 (segment (start 145.732 101.6) (end 145.288 101.156) (width 0.35) (layer F.Cu) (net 5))
 (segment (start 172.974 106.141002) (end 172.974 97.282) (width 0.35) (layer F.Cu) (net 6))
 (segment (start 172.974 97.282) (end 170.688 94.996) (width 0.35) (layer F.Cu) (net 6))
 (segment (start 148.844 108.712) (end 147.478 108.712) (width 0.35) (layer F.Cu) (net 6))
 (segment (start 147.302999 108.887001) (end 147.302999 111.991681) (width 0.35) (layer F.Cu) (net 6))
 (segment (start 147.478 108.712) (end 147.302999 108.887001) (width 0.35) (layer F.Cu) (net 6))
 (segment (start 147.302999 111.991681) (end 148.818319 113.507001) (width 0.35) (layer F.Cu) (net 6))
 (segment (start 148.818319 113.507001) (end 165.608001 113.507001) (width 0.35) (layer F.Cu) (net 6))
 (segment (start 165.608001 113.507001) (end 172.974 106.141002) (width 0.35) (layer F.Cu) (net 6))
 (segment (start 145.288 107.696) (end 147.828 107.696) (width 0.35) (layer F.Cu) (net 6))
 (segment (start 147.828 107.696) (end 148.844 108.712) (width 0.35) (layer F.Cu) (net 6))
 (segment (start 153.162 108.712) (end 154.528 108.712) (width 0.35) (layer F.Cu) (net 8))
 (segment (start 154.528 108.712) (end 156.306 106.934) (width 0.35) (layer F.Cu) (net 8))
 (segment (start 156.306 106.934) (end 156.39594 106.934) (width 0.35) (layer F.Cu) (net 8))
 (segment (start 156.39594 106.934) (end 158.496 106.934) (width 0.35) (layer F.Cu) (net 8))
 (segment (start 153.3144 108.712) (end 153.162 108.712) (width 0.35) (layer F.Cu) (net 8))
 (segment (start 159.39643 106.934) (end 158.496 106.934) (width 0.35) (layer F.Cu) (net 8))
 (segment (start 155.702 101.346) (end 156.67228 100.37572) (width 0.35) (layer F.Cu) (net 9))
 (segment (start 156.67228 100.37572) (end 158.308 100.37572) (width 0.35) (layer F.Cu) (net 9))
 (segment (start 155.702 103.7844) (end 155.702 101.346) (width 0.35) (layer F.Cu) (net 9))
 (segment (start 153.162 106.172) (end 153.3144 106.172) (width 0.35) (layer F.Cu) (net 9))
 (segment (start 153.3144 106.172) (end 155.702 103.7844) (width 0.35) (layer F.Cu) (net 9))
 (segment (start 153.162 102.4184) (end 153.162 103.632) (width 0.35) (layer F.Cu) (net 10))
 (segment (start 153.162 97.066996) (end 153.162 102.4184) (width 0.35) (layer F.Cu) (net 10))
 (segment (start 155.972136 94.25686) (end 153.162 97.066996) (width 0.35) (layer F.Cu) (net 10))
 (segment (start 158.242 94.25686) (end 155.972136 94.25686) (width 0.35) (layer F.Cu) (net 10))
 (segment (start 165.1 89.916) (end 165.1 100.584) (width 0.35) (layer B.Cu) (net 7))
 (segment (start 165.1 100.584) (end 163.426 100.584) (width 0.35) (layer F.Cu) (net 7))
 (segment (start 161.544 102.466) (end 161.544 102.616) (width 0.35) (layer F.Cu) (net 7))
 (segment (start 163.426 100.584) (end 161.544 102.466) (width 0.35) (layer F.Cu) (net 7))
 (via (at 165.1 100.584) (size 1.3) (drill 0.8) (layers F.Cu B.Cu) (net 7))
 (segment (start 170.688 92.456) (end 168.148 89.916) (width 0.35) (layer F.Cu) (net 7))
 (via (at 165.1 89.916) (size 1.3) (drill 0.8) (layers F.Cu B.Cu) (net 7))
 (segment (start 168.148 89.916) (end 165.1 89.916) (width 0.35) (layer F.Cu) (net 7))
 (segment (start 159.258 103.378) (end 160.782 103.378) (width 0.35) (layer F.Cu) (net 7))
 (segment (start 160.782 103.378) (end 161.544 102.616) (width 0.35) (layer F.Cu) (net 7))
 (segment (start 163.817311 96.029846) (end 163.817311 94.371311) (width 0.35) (layer F.Cu) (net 1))
 (segment (start 163.817311 94.371311) (end 161.544 92.098) (width 0.35) (layer F.Cu) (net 1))
 (segment (start 161.544 92.098) (end 161.544 91.948) (width 0.35) (layer F.Cu) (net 1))
 (segment (start 161.798 91.948) (end 161.544 91.948) (width 0.35) (layer F.Cu) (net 1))
 (segment (start 165.932481 99.074081) (end 163.817311 99.074081) (width 0.35) (layer F.Cu) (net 1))
 (segment (start 166.9344 100.076) (end 165.932481 99.074081) (width 0.35) (layer F.Cu) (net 1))
 (segment (start 168.148 100.076) (end 166.9344 100.076) (width 0.35) (layer F.Cu) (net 1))
 (segment (start 163.817311 96.029846) (end 163.817311 99.074081) (width 0.35) (layer B.Cu) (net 1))
 (via (at 163.817311 99.074081) (size 1.3) (drill 0.8) (layers F.Cu B.Cu) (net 1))
 (via (at 163.817311 96.029846) (size 1.3) (drill 0.8) (layers F.Cu B.Cu) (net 1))
 (segment (start 159.192 97.25914) (end 159.192 93.1) (width 0.35) (layer F.Cu) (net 1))
 (segment (start 159.192 93.1) (end 160.344 91.948) (width 0.35) (layer F.Cu) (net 1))
 (segment (start 160.344 91.948) (end 161.544 91.948) (width 0.35) (layer F.Cu) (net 1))
 (segment (start 170.688 97.536) (end 171.909314 97.536) (width 0.35) (layer F.Cu) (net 4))
 (segment (start 171.909314 97.536) (end 172.076601 97.703287) (width 0.35) (layer F.Cu) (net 4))
 (segment (start 172.076601 97.703287) (end 172.076601 101.519399) (width 0.35) (layer F.Cu) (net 4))
 (segment (start 172.076601 101.519399) (end 171.164 102.432) (width 0.35) (layer F.Cu) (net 4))
 (segment (start 171.164 102.432) (end 171.164 103.632) (width 0.35) (layer F.Cu) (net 4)))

